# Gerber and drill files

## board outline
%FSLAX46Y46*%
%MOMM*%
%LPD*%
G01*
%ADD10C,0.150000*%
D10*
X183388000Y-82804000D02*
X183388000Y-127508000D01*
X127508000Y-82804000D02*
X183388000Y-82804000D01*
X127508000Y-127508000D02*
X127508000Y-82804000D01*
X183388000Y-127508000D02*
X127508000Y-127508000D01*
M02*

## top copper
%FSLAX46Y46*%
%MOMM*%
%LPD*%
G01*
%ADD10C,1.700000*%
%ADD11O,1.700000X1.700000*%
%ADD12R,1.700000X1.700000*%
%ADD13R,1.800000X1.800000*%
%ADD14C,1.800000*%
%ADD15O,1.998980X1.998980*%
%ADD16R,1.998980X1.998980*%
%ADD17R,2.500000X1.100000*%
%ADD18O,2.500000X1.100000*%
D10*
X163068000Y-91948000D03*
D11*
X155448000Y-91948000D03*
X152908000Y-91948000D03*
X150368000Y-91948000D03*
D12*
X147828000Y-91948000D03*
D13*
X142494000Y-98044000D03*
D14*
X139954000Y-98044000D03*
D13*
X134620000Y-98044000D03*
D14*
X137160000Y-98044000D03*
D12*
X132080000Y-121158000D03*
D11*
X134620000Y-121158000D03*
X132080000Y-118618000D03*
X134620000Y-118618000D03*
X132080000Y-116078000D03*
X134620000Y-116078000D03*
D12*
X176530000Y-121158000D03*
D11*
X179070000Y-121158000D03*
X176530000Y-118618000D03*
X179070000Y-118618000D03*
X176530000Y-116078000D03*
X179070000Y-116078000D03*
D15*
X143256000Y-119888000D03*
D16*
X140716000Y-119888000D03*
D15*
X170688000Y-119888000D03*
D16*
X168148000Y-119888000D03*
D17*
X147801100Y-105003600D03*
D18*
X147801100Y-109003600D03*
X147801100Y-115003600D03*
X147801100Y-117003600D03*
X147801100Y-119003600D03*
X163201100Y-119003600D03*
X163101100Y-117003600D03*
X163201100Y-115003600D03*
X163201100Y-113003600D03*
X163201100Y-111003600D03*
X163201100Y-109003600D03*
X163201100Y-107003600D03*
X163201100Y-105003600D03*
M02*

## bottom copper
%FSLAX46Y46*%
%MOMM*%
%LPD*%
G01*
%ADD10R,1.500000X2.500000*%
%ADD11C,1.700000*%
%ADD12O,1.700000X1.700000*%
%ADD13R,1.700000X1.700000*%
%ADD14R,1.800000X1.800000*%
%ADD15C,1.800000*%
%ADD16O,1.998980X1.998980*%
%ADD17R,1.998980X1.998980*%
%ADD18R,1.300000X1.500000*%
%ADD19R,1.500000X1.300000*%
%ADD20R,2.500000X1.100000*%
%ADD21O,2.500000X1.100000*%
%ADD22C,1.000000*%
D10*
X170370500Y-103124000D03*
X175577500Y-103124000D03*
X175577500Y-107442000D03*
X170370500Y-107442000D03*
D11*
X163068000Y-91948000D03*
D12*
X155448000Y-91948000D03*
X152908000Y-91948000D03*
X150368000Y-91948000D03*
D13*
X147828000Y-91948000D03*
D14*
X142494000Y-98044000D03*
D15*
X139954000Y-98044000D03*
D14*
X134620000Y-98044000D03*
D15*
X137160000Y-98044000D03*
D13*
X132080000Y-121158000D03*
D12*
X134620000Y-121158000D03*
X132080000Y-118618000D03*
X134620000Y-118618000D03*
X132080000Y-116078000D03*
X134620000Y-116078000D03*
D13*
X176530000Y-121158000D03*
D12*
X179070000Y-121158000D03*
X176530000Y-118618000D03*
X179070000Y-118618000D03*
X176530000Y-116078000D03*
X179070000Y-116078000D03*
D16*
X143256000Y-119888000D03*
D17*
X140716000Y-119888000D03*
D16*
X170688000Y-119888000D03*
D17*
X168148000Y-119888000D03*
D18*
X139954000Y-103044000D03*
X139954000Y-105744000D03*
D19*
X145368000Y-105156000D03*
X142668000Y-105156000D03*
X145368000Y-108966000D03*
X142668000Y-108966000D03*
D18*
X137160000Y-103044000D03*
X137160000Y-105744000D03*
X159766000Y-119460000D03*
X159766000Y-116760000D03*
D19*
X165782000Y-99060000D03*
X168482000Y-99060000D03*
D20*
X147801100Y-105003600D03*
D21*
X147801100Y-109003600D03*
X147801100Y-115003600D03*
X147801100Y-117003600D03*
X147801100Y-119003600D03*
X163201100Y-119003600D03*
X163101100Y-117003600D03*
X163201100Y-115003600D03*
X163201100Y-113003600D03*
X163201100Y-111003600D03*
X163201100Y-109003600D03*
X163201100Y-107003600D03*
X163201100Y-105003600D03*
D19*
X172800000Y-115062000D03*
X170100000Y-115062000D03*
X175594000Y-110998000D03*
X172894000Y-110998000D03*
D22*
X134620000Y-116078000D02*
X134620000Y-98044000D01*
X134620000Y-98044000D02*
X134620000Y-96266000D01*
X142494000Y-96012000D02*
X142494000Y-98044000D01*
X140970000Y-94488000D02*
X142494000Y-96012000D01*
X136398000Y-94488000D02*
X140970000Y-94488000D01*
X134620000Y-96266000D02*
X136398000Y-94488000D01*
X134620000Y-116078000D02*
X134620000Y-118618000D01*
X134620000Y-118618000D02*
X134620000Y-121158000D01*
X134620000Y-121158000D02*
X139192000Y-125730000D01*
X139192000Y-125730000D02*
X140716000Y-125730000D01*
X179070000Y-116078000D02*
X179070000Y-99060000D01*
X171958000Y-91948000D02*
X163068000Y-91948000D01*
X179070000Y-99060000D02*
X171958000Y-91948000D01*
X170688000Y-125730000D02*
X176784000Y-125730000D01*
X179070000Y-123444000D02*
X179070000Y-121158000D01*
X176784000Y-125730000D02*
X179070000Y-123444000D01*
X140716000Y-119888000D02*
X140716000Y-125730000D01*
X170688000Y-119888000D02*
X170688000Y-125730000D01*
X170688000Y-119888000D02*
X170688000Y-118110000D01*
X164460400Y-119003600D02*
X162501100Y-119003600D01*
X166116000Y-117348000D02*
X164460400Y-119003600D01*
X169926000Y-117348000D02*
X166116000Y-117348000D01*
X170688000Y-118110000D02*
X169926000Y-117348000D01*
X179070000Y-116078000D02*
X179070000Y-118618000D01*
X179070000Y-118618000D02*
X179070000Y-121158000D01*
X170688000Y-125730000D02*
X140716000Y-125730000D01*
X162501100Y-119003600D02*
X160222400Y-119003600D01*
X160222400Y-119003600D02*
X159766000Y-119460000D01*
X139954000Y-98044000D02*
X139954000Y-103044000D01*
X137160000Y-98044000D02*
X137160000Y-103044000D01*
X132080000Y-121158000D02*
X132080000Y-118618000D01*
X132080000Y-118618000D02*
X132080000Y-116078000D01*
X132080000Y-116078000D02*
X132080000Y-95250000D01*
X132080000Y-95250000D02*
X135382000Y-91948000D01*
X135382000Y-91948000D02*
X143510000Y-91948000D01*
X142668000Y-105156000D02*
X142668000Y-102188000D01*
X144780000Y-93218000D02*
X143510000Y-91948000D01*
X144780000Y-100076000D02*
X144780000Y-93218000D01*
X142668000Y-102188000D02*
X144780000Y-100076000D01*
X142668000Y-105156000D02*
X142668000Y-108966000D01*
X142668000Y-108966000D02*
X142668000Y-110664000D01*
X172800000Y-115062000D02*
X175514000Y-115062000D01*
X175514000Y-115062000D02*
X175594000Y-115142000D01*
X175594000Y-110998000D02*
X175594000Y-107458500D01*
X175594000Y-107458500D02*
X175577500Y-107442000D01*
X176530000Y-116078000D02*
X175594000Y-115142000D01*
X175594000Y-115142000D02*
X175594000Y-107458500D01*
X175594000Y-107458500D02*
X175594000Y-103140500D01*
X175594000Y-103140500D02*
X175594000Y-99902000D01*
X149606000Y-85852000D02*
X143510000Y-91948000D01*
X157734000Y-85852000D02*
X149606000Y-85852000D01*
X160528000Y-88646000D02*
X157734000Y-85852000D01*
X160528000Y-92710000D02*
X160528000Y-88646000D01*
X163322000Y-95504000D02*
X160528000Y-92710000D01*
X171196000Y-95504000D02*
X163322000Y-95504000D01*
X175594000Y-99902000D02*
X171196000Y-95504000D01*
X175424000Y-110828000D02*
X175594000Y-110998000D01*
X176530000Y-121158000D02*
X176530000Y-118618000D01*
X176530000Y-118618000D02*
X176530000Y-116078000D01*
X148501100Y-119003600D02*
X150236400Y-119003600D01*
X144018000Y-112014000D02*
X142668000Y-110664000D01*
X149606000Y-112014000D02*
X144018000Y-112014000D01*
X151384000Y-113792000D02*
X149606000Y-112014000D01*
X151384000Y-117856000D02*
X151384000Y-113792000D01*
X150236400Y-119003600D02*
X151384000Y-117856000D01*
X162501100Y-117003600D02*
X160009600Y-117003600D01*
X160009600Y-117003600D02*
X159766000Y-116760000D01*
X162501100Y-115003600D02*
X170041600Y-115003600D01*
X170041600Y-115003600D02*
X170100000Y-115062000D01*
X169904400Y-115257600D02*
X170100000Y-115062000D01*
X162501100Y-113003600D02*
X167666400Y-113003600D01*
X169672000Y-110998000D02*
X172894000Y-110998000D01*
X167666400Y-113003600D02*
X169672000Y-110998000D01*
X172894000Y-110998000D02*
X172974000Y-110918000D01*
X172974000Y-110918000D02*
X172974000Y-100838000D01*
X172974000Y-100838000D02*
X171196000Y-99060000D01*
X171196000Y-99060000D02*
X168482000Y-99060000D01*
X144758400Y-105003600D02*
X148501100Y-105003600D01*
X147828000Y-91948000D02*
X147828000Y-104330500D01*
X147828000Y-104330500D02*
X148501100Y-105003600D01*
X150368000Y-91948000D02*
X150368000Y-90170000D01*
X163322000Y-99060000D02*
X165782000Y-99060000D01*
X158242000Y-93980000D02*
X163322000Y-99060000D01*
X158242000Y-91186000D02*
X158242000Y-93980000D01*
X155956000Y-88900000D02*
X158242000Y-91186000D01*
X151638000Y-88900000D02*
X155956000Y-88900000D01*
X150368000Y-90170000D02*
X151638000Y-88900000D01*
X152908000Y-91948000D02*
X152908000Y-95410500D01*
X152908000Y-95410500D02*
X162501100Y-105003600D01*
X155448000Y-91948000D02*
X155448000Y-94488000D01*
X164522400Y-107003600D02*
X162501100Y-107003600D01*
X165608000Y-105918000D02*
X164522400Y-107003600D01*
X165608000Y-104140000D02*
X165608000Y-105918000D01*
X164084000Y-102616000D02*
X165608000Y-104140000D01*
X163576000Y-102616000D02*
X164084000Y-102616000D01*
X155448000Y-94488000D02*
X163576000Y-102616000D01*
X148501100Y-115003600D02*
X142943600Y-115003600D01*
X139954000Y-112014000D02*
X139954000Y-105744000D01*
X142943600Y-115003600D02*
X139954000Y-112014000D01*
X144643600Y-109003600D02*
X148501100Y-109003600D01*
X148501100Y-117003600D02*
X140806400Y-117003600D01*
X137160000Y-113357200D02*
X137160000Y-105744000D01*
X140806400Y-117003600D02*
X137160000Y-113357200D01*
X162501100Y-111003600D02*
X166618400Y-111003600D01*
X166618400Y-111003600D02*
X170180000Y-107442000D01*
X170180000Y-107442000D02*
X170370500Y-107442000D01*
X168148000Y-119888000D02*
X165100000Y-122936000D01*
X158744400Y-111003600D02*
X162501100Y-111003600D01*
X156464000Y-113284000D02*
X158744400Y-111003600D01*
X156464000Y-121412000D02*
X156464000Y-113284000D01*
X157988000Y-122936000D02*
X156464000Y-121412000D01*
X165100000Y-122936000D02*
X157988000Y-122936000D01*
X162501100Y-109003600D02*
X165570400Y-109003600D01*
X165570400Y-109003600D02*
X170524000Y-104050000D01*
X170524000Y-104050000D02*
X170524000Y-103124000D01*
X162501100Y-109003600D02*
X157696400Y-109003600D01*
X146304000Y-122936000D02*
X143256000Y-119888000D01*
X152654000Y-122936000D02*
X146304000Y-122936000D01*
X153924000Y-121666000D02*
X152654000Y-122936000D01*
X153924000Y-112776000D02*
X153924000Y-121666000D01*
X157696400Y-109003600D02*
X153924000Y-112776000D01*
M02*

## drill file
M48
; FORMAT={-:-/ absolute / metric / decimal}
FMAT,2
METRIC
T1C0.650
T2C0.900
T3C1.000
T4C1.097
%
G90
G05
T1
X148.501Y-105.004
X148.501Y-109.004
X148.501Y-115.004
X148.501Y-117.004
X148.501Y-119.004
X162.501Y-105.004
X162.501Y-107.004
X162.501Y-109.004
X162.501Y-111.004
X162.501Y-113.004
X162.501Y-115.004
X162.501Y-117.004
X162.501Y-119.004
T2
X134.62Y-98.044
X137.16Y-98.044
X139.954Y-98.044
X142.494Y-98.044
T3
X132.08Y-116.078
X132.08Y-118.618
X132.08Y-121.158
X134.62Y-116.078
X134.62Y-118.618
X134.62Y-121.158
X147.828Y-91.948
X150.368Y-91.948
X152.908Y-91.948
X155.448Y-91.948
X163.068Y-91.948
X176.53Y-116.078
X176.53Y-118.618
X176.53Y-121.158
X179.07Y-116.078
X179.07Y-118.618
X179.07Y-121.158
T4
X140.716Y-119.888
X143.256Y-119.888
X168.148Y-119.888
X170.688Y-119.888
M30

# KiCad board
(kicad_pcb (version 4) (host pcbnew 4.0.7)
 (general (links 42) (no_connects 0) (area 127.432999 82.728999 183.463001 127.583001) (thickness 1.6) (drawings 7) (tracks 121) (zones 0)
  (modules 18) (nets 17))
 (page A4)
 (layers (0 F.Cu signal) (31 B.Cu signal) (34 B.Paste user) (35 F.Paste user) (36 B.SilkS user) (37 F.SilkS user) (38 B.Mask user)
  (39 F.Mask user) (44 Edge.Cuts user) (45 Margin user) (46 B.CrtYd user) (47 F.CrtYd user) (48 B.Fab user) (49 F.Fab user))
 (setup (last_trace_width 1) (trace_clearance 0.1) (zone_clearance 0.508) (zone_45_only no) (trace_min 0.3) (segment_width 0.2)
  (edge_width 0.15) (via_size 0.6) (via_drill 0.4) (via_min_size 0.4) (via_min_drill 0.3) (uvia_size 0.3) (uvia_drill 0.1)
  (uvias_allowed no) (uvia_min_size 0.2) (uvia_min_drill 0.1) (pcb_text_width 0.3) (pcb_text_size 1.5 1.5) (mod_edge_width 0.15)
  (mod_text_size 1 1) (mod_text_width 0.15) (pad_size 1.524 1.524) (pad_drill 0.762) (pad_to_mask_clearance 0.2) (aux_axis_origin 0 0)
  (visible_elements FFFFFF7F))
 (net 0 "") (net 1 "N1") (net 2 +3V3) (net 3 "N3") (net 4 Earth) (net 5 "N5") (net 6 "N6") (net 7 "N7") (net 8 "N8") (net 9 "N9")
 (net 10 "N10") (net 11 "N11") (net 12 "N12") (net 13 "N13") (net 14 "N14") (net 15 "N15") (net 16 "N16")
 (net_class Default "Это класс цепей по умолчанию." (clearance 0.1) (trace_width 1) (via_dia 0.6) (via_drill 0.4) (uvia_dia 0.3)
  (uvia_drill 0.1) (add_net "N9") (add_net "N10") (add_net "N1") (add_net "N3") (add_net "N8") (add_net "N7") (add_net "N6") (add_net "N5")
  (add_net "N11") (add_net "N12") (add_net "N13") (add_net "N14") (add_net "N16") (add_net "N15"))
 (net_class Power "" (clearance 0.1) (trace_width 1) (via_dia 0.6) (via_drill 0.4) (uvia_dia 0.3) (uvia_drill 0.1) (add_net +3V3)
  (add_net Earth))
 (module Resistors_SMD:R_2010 (layer B.Cu) (at 172.974 103.124)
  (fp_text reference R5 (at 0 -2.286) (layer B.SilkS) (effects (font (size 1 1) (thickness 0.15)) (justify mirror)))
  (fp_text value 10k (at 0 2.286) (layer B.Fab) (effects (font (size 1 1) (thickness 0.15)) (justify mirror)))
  (pad 1 smd rect (at -2.6035 0) (size 1.5 2.5) (layers B.Cu B.Paste B.Mask) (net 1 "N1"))
  (pad 2 smd rect (at 2.6035 0) (size 1.5 2.5) (layers B.Cu B.Paste B.Mask) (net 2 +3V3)))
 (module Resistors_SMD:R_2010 (layer B.Cu) (at 172.974 107.442 180)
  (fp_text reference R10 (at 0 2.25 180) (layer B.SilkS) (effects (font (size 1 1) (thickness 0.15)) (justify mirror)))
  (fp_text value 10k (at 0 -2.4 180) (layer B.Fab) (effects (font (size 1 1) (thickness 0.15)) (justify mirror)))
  (pad 1 smd rect (at -2.6035 0 180) (size 1.5 2.5) (layers B.Cu B.Paste B.Mask) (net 2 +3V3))
  (pad 2 smd rect (at 2.6035 0 180) (size 1.5 2.5) (layers B.Cu B.Paste B.Mask) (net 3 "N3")))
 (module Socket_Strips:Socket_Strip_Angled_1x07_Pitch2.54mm (layer F.Cu) (at 163.068 91.948 270)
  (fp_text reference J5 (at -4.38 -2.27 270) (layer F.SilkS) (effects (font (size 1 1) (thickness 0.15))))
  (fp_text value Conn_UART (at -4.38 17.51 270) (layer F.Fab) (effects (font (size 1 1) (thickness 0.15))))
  (pad 7 thru_hole circle (at 0 0 270) (size 1.7 1.7) (drill 1) (layers *.Cu *.Mask) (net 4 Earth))
  (pad 4 thru_hole oval (at 0 7.62 270) (size 1.7 1.7) (drill 1) (layers *.Cu *.Mask) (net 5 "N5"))
  (pad 3 thru_hole oval (at 0 10.16 270) (size 1.7 1.7) (drill 1) (layers *.Cu *.Mask) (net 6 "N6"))
  (pad 2 thru_hole oval (at 0 12.7 270) (size 1.7 1.7) (drill 1) (layers *.Cu *.Mask) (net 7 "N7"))
  (pad 1 thru_hole rect (at 0 15.24 270) (size 1.7 1.7) (drill 1) (layers *.Cu *.Mask) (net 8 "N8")))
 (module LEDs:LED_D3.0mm (layer F.Cu) (at 142.494 98.044 180)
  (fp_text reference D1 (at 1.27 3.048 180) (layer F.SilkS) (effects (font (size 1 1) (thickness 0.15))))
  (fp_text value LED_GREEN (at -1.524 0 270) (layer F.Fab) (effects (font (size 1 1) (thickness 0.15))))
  (pad 1 thru_hole rect (at 0 0 180) (size 1.8 1.8) (drill 0.9) (layers *.Cu *.Mask) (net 4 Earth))
  (pad 2 thru_hole circle (at 2.54 0 180) (size 1.8 1.8) (drill 0.9) (layers *.Cu *.Mask) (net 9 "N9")))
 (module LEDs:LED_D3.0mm (layer F.Cu) (at 134.62 98.044)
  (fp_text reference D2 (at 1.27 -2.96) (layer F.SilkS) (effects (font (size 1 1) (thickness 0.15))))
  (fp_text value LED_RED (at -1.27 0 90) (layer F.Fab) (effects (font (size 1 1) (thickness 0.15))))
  (pad 1 thru_hole rect (at 0 0) (size 1.8 1.8) (drill 0.9) (layers *.Cu *.Mask) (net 4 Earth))
  (pad 2 thru_hole circle (at 2.54 0) (size 1.8 1.8) (drill 0.9) (layers *.Cu *.Mask) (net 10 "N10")))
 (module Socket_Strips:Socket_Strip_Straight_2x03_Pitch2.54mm (layer F.Cu) (at 132.08 121.158 180)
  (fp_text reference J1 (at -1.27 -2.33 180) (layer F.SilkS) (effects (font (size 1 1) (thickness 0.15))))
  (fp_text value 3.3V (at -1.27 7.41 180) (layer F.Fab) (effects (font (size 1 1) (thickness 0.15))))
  (pad 1 thru_hole rect (at 0 0 180) (size 1.7 1.7) (drill 1) (layers *.Cu *.Mask) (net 2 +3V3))
  (pad 2 thru_hole oval (at -2.54 0 180) (size 1.7 1.7) (drill 1) (layers *.Cu *.Mask) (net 4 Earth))
  (pad 3 thru_hole oval (at 0 2.54 180) (size 1.7 1.7) (drill 1) (layers *.Cu *.Mask) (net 2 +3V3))
  (pad 4 thru_hole oval (at -2.54 2.54 180) (size 1.7 1.7) (drill 1) (layers *.Cu *.Mask) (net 4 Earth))
  (pad 5 thru_hole oval (at 0 5.08 180) (size 1.7 1.7) (drill 1) (layers *.Cu *.Mask) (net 2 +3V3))
  (pad 6 thru_hole oval (at -2.54 5.08 180) (size 1.7 1.7) (drill 1) (layers *.Cu *.Mask) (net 4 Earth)))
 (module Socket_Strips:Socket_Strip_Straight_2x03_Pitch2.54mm (layer F.Cu) (at 176.53 121.158 180)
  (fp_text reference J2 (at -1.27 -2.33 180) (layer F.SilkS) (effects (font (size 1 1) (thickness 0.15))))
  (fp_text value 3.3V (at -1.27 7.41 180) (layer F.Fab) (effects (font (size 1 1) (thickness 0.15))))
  (pad 1 thru_hole rect (at 0 0 180) (size 1.7 1.7) (drill 1) (layers *.Cu *.Mask) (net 2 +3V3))
  (pad 2 thru_hole oval (at -2.54 0 180) (size 1.7 1.7) (drill 1) (layers *.Cu *.Mask) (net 4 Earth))
  (pad 3 thru_hole oval (at 0 2.54 180) (size 1.7 1.7) (drill 1) (layers *.Cu *.Mask) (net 2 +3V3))
  (pad 4 thru_hole oval (at -2.54 2.54 180) (size 1.7 1.7) (drill 1) (layers *.Cu *.Mask) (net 4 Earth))
  (pad 5 thru_hole oval (at 0 5.08 180) (size 1.7 1.7) (drill 1) (layers *.Cu *.Mask) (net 2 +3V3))
  (pad 6 thru_hole oval (at -2.54 5.08 180) (size 1.7 1.7) (drill 1) (layers *.Cu *.Mask) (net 4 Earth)))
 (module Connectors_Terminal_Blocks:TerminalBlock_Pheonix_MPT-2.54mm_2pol (layer F.Cu) (at 140.716 119.888)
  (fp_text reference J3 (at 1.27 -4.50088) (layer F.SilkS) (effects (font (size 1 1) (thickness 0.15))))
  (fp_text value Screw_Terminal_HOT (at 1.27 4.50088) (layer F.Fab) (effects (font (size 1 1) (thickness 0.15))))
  (pad 2 thru_hole oval (at 2.54 0) (size 1.99898 1.99898) (drill 1.09728) (layers *.Cu *.Mask) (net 1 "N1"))
  (pad 1 thru_hole rect (at 0 0) (size 1.99898 1.99898) (drill 1.09728) (layers *.Cu *.Mask) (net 4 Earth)))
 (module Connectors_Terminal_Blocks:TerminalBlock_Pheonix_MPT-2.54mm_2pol (layer F.Cu) (at 168.148 119.888)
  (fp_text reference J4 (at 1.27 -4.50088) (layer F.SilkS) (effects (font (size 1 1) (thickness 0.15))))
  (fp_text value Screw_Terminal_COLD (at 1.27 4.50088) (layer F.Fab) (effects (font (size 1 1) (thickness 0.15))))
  (pad 2 thru_hole oval (at 2.54 0) (size 1.99898 1.99898) (drill 1.09728) (layers *.Cu *.Mask) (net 4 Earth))
  (pad 1 thru_hole rect (at 0 0) (size 1.99898 1.99898) (drill 1.09728) (layers *.Cu *.Mask) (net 3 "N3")))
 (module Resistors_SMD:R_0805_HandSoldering (layer B.Cu) (at 139.954 104.394 270)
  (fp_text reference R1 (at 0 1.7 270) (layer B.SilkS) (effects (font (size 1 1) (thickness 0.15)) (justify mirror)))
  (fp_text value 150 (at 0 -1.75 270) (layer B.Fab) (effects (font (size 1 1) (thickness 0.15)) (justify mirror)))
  (pad 1 smd rect (at -1.35 0 270) (size 1.5 1.3) (layers B.Cu B.Paste B.Mask) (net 9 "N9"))
  (pad 2 smd rect (at 1.35 0 270) (size 1.5 1.3) (layers B.Cu B.Paste B.Mask) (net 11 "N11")))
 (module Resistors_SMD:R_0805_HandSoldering (layer B.Cu) (at 144.018 105.156 180)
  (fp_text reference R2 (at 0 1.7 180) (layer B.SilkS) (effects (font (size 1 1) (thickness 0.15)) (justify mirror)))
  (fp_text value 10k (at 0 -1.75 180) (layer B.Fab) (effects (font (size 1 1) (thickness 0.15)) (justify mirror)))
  (pad 1 smd rect (at -1.35 0 180) (size 1.5 1.3) (layers B.Cu B.Paste B.Mask) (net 8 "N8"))
  (pad 2 smd rect (at 1.35 0 180) (size 1.5 1.3) (layers B.Cu B.Paste B.Mask) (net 2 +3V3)))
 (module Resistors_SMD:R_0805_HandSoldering (layer B.Cu) (at 144.018 108.966 180)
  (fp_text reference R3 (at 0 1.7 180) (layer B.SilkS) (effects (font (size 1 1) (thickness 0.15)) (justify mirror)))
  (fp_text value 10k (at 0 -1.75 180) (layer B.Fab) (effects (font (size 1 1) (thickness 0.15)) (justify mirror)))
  (pad 1 smd rect (at -1.35 0 180) (size 1.5 1.3) (layers B.Cu B.Paste B.Mask) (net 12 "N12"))
  (pad 2 smd rect (at 1.35 0 180) (size 1.5 1.3) (layers B.Cu B.Paste B.Mask) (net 2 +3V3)))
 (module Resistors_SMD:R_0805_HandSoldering (layer B.Cu) (at 137.16 104.394 270)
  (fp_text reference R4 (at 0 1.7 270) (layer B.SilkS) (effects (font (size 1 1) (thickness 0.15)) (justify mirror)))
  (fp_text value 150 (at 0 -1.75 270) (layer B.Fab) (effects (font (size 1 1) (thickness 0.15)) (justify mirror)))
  (pad 1 smd rect (at -1.35 0 270) (size 1.5 1.3) (layers B.Cu B.Paste B.Mask) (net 10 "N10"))
  (pad 2 smd rect (at 1.35 0 270) (size 1.5 1.3) (layers B.Cu B.Paste B.Mask) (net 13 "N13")))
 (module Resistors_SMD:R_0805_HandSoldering (layer B.Cu) (at 159.766 118.11 90)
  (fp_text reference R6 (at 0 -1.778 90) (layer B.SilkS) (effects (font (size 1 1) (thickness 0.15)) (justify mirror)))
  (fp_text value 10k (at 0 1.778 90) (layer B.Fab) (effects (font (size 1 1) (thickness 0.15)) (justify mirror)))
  (pad 1 smd rect (at -1.35 0 90) (size 1.5 1.3) (layers B.Cu B.Paste B.Mask) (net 4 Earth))
  (pad 2 smd rect (at 1.35 0 90) (size 1.5 1.3) (layers B.Cu B.Paste B.Mask) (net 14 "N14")))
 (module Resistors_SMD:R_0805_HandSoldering (layer B.Cu) (at 167.132 99.06)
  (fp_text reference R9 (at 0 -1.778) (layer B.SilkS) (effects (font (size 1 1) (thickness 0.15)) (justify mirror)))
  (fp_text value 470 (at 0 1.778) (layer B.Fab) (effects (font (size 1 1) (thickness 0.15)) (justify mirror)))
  (pad 1 smd rect (at -1.35 0) (size 1.5 1.3) (layers B.Cu B.Paste B.Mask) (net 7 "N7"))
  (pad 2 smd rect (at 1.35 0) (size 1.5 1.3) (layers B.Cu B.Paste B.Mask) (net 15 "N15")))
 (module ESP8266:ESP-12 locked (layer F.Cu) (at 148.5011 105.0036)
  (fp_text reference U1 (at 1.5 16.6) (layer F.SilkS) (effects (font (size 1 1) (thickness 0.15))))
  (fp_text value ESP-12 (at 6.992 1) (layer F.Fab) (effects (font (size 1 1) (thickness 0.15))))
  (pad 1 thru_hole rect (at 0 0) (size 2.5 1.1) (drill 0.65 (offset -0.7 0)) (layers *.Cu *.Mask F.SilkS) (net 8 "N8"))
  (pad 3 thru_hole oval (at 0 4) (size 2.5 1.1) (drill 0.65 (offset -0.7 0)) (layers *.Cu *.Mask F.SilkS) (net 12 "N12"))
  (pad 6 thru_hole oval (at 0 10) (size 2.5 1.1) (drill 0.65 (offset -0.7 0)) (layers *.Cu *.Mask F.SilkS) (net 11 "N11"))
  (pad 7 thru_hole oval (at 0 12) (size 2.5 1.1) (drill 0.65 (offset -0.7 0)) (layers *.Cu *.Mask F.SilkS) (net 13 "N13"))
  (pad 8 thru_hole oval (at 0 14) (size 2.5 1.1) (drill 0.65 (offset -0.7 0)) (layers *.Cu *.Mask F.SilkS) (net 2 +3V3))
  (pad 9 thru_hole oval (at 14 14) (size 2.5 1.1) (drill 0.65 (offset 0.7 0)) (layers *.Cu *.Mask F.SilkS) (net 4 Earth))
  (pad 10 thru_hole oval (at 14 12) (size 2.5 1.1) (drill 0.65 (offset 0.6 0)) (layers *.Cu *.Mask F.SilkS) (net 14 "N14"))
  (pad 11 thru_hole oval (at 14 10) (size 2.5 1.1) (drill 0.65 (offset 0.7 0)) (layers *.Cu *.Mask F.SilkS) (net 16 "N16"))
  (pad 12 thru_hole oval (at 14 8) (size 2.5 1.1) (drill 0.65 (offset 0.7 0)) (layers *.Cu *.Mask F.SilkS) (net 15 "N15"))
  (pad 13 thru_hole oval (at 14 6) (size 2.5 1.1) (drill 0.65 (offset 0.7 0)) (layers *.Cu *.Mask F.SilkS) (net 3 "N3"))
  (pad 14 thru_hole oval (at 14 4) (size 2.5 1.1) (drill 0.65 (offset 0.7 0)) (layers *.Cu *.Mask F.SilkS) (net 1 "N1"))
  (pad 15 thru_hole oval (at 14 2) (size 2.5 1.1) (drill 0.65 (offset 0.7 0)) (layers *.Cu *.Mask F.SilkS) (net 5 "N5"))
  (pad 16 thru_hole oval (at 14 0) (size 2.5 1.1) (drill 0.65 (offset 0.7 0)) (layers *.Cu *.Mask F.SilkS) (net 6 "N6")))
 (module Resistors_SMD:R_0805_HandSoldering (layer B.Cu) (at 171.45 115.062 180)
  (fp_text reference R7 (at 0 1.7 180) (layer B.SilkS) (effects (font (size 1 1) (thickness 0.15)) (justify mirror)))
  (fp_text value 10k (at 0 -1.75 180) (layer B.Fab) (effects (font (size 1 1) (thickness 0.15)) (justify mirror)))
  (pad 1 smd rect (at -1.35 0 180) (size 1.5 1.3) (layers B.Cu B.Paste B.Mask) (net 2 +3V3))
  (pad 2 smd rect (at 1.35 0 180) (size 1.5 1.3) (layers B.Cu B.Paste B.Mask) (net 16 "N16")))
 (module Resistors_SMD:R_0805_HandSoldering (layer B.Cu) (at 174.244 110.998 180)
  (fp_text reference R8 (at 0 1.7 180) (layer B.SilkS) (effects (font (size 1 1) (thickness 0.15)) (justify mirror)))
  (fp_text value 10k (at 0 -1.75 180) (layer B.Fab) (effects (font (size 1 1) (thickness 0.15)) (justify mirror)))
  (pad 1 smd rect (at -1.35 0 180) (size 1.5 1.3) (layers B.Cu B.Paste B.Mask) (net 2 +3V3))
  (pad 2 smd rect (at 1.35 0 180) (size 1.5 1.3) (layers B.Cu B.Paste B.Mask) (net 15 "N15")))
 (gr_line (start 183.388 82.804) (end 183.388 127.508) (angle 90) (layer Edge.Cuts) (width 0.15))
 (gr_line (start 127.508 82.804) (end 183.388 82.804) (angle 90) (layer Edge.Cuts) (width 0.15))
 (gr_line (start 127.508 127.508) (end 127.508 82.804) (angle 90) (layer Edge.Cuts) (width 0.15))
 (gr_line (start 183.388 127.508) (end 127.508 127.508) (angle 90) (layer Edge.Cuts) (width 0.15))
 (segment (start 134.62 116.078) (end 134.62 98.044) (width 1) (layer B.Cu) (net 4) (status 30))
 (segment (start 134.62 98.044) (end 134.62 96.266) (width 1) (layer B.Cu) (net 4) (status 10))
 (segment (start 142.494 96.012) (end 142.494 98.044) (width 1) (layer B.Cu) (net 4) (status 20))
 (segment (start 140.97 94.488) (end 142.494 96.012) (width 1) (layer B.Cu) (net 4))
 (segment (start 136.398 94.488) (end 140.97 94.488) (width 1) (layer B.Cu) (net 4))
 (segment (start 134.62 96.266) (end 136.398 94.488) (width 1) (layer B.Cu) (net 4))
 (segment (start 134.62 116.078) (end 134.62 118.618) (width 1) (layer B.Cu) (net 4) (status 30))
 (segment (start 134.62 118.618) (end 134.62 121.158) (width 1) (layer B.Cu) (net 4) (status 30))
 (segment (start 134.62 121.158) (end 139.192 125.73) (width 1) (layer B.Cu) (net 4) (status 10))
 (segment (start 139.192 125.73) (end 140.716 125.73) (width 1) (layer B.Cu) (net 4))
 (segment (start 179.07 116.078) (end 179.07 99.06) (width 1) (layer B.Cu) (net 4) (status 10))
 (segment (start 171.958 91.948) (end 163.068 91.948) (width 1) (layer B.Cu) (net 4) (status 20))
 (segment (start 179.07 99.06) (end 171.958 91.948) (width 1) (layer B.Cu) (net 4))
 (segment (start 170.688 125.73) (end 176.784 125.73) (width 1) (layer B.Cu) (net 4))
 (segment (start 179.07 123.444) (end 179.07 121.158) (width 1) (layer B.Cu) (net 4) (status 20))
 (segment (start 176.784 125.73) (end 179.07 123.444) (width 1) (layer B.Cu) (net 4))
 (segment (start 140.716 119.888) (end 140.716 125.73) (width 1) (layer B.Cu) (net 4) (status 10))
 (segment (start 170.688 119.888) (end 170.688 125.73) (width 1) (layer B.Cu) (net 4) (status 10))
 (segment (start 170.688 119.888) (end 170.688 118.11) (width 1) (layer B.Cu) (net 4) (status 10))
 (segment (start 164.4604 119.0036) (end 162.5011 119.0036) (width 1) (layer B.Cu) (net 4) (status 20))
 (segment (start 166.116 117.348) (end 164.4604 119.0036) (width 1) (layer B.Cu) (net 4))
 (segment (start 169.926 117.348) (end 166.116 117.348) (width 1) (layer B.Cu) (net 4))
 (segment (start 170.688 118.11) (end 169.926 117.348) (width 1) (layer B.Cu) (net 4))
 (segment (start 179.07 116.078) (end 179.07 118.618) (width 1) (layer B.Cu) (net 4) (status 30))
 (segment (start 179.07 118.618) (end 179.07 121.158) (width 1) (layer B.Cu) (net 4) (status 30))
 (segment (start 170.688 125.73) (end 140.716 125.73) (width 1) (layer B.Cu) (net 4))
 (segment (start 162.5011 119.0036) (end 160.2224 119.0036) (width 1) (layer B.Cu) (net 4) (status 30))
 (segment (start 160.2224 119.0036) (end 159.766 119.46) (width 1) (layer B.Cu) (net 4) (status 30))
 (segment (start 139.954 98.044) (end 139.954 103.044) (width 1) (layer B.Cu) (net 9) (status 30))
 (segment (start 137.16 98.044) (end 137.16 103.044) (width 1) (layer B.Cu) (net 10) (status 30))
 (segment (start 132.08 121.158) (end 132.08 118.618) (width 1) (layer B.Cu) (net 2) (status 30))
 (segment (start 132.08 118.618) (end 132.08 116.078) (width 1) (layer B.Cu) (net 2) (status 30))
 (segment (start 132.08 116.078) (end 132.08 95.25) (width 1) (layer B.Cu) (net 2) (status 10))
 (segment (start 132.08 95.25) (end 135.382 91.948) (width 1) (layer B.Cu) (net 2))
 (segment (start 135.382 91.948) (end 143.51 91.948) (width 1) (layer B.Cu) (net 2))
 (segment (start 142.668 105.156) (end 142.668 102.188) (width 1) (layer B.Cu) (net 2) (status 10))
 (segment (start 144.78 93.218) (end 143.51 91.948) (width 1) (layer B.Cu) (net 2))
 (segment (start 144.78 100.076) (end 144.78 93.218) (width 1) (layer B.Cu) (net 2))
 (segment (start 142.668 102.188) (end 144.78 100.076) (width 1) (layer B.Cu) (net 2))
 (segment (start 142.668 105.156) (end 142.668 108.966) (width 1) (layer B.Cu) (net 2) (status 30))
 (segment (start 142.668 108.966) (end 142.668 110.664) (width 1) (layer B.Cu) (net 2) (status 10))
 (segment (start 172.8 115.062) (end 175.514 115.062) (width 1) (layer B.Cu) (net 2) (status 10))
 (segment (start 175.514 115.062) (end 175.594 115.142) (width 1) (layer B.Cu) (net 2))
 (segment (start 175.594 110.998) (end 175.594 107.4585) (width 1) (layer B.Cu) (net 2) (status 30))
 (segment (start 175.594 107.4585) (end 175.5775 107.442) (width 1) (layer B.Cu) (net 2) (status 30))
 (segment (start 176.53 116.078) (end 175.594 115.142) (width 1) (layer B.Cu) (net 2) (status 10))
 (segment (start 175.594 115.142) (end 175.594 107.4585) (width 1) (layer B.Cu) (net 2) (status 20))
 (segment (start 175.594 107.4585) (end 175.594 103.1405) (width 1) (layer B.Cu) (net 2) (status 30))
 (segment (start 175.594 103.1405) (end 175.594 99.902) (width 1) (layer B.Cu) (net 2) (status 10))
 (segment (start 149.606 85.852) (end 143.51 91.948) (width 1) (layer B.Cu) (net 2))
 (segment (start 157.734 85.852) (end 149.606 85.852) (width 1) (layer B.Cu) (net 2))
 (segment (start 160.528 88.646) (end 157.734 85.852) (width 1) (layer B.Cu) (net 2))
 (segment (start 160.528 92.71) (end 160.528 88.646) (width 1) (layer B.Cu) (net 2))
 (segment (start 163.322 95.504) (end 160.528 92.71) (width 1) (layer B.Cu) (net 2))
 (segment (start 171.196 95.504) (end 163.322 95.504) (width 1) (layer B.Cu) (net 2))
 (segment (start 175.594 99.902) (end 171.196 95.504) (width 1) (layer B.Cu) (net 2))
 (segment (start 175.424 110.828) (end 175.594 110.998) (width 1) (layer B.Cu) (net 2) (status 30))
 (segment (start 176.53 121.158) (end 176.53 118.618) (width 1) (layer B.Cu) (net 2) (status 30))
 (segment (start 176.53 118.618) (end 176.53 116.078) (width 1) (layer B.Cu) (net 2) (status 30))
 (segment (start 148.5011 119.0036) (end 150.2364 119.0036) (width 1) (layer B.Cu) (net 2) (status 10))
 (segment (start 144.018 112.014) (end 142.668 110.664) (width 1) (layer B.Cu) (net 2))
 (segment (start 149.606 112.014) (end 144.018 112.014) (width 1) (layer B.Cu) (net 2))
 (segment (start 151.384 113.792) (end 149.606 112.014) (width 1) (layer B.Cu) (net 2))
 (segment (start 151.384 117.856) (end 151.384 113.792) (width 1) (layer B.Cu) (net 2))
 (segment (start 150.2364 119.0036) (end 151.384 117.856) (width 1) (layer B.Cu) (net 2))
 (segment (start 162.5011 117.0036) (end 160.0096 117.0036) (width 1) (layer B.Cu) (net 14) (status 30))
 (segment (start 160.0096 117.0036) (end 159.766 116.76) (width 1) (layer B.Cu) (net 14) (status 30))
 (segment (start 162.5011 115.0036) (end 170.0416 115.0036) (width 1) (layer B.Cu) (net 16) (status 30))
 (segment (start 170.0416 115.0036) (end 170.1 115.062) (width 1) (layer B.Cu) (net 16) (status 30))
 (segment (start 169.9044 115.2576) (end 170.1 115.062) (width 1) (layer B.Cu) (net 16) (status 30))
 (segment (start 162.5011 113.0036) (end 167.6664 113.0036) (width 1) (layer B.Cu) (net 15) (status 10))
 (segment (start 169.672 110.998) (end 172.894 110.998) (width 1) (layer B.Cu) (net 15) (status 20))
 (segment (start 167.6664 113.0036) (end 169.672 110.998) (width 1) (layer B.Cu) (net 15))
 (segment (start 172.894 110.998) (end 172.974 110.918) (width 1) (layer B.Cu) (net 15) (status 30))
 (segment (start 172.974 110.918) (end 172.974 100.838) (width 1) (layer B.Cu) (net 15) (status 10))
 (segment (start 172.974 100.838) (end 171.196 99.06) (width 1) (layer B.Cu) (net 15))
 (segment (start 171.196 99.06) (end 168.482 99.06) (width 1) (layer B.Cu) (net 15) (status 20))
 (segment (start 144.7584 105.0036) (end 148.5011 105.0036) (width 1) (layer B.Cu) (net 8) (status 30))
 (segment (start 147.828 91.948) (end 147.828 104.3305) (width 1) (layer B.Cu) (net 8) (status 10))
 (segment (start 147.828 104.3305) (end 148.5011 105.0036) (width 1) (layer B.Cu) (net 8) (status 20))
 (segment (start 150.368 91.948) (end 150.368 90.17) (width 1) (layer B.Cu) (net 7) (status 10))
 (segment (start 163.322 99.06) (end 165.782 99.06) (width 1) (layer B.Cu) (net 7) (status 20))
 (segment (start 158.242 93.98) (end 163.322 99.06) (width 1) (layer B.Cu) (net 7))
 (segment (start 158.242 91.186) (end 158.242 93.98) (width 1) (layer B.Cu) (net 7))
 (segment (start 155.956 88.9) (end 158.242 91.186) (width 1) (layer B.Cu) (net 7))
 (segment (start 151.638 88.9) (end 155.956 88.9) (width 1) (layer B.Cu) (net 7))
 (segment (start 150.368 90.17) (end 151.638 88.9) (width 1) (layer B.Cu) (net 7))
 (segment (start 152.908 91.948) (end 152.908 95.4105) (width 1) (layer B.Cu) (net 6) (status 10))
 (segment (start 152.908 95.4105) (end 162.5011 105.0036) (width 1) (layer B.Cu) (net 6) (status 20))
 (segment (start 155.448 91.948) (end 155.448 94.488) (width 1) (layer B.Cu) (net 5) (status 10))
 (segment (start 164.5224 107.0036) (end 162.5011 107.0036) (width 1) (layer B.Cu) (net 5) (status 20))
 (segment (start 165.608 105.918) (end 164.5224 107.0036) (width 1) (layer B.Cu) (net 5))
 (segment (start 165.608 104.14) (end 165.608 105.918) (width 1) (layer B.Cu) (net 5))
 (segment (start 164.084 102.616) (end 165.608 104.14) (width 1) (layer B.Cu) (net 5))
 (segment (start 163.576 102.616) (end 164.084 102.616) (width 1) (layer B.Cu) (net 5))
 (segment (start 155.448 94.488) (end 163.576 102.616) (width 1) (layer B.Cu) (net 5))
 (segment (start 148.5011 115.0036) (end 142.9436 115.0036) (width 1) (layer B.Cu) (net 11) (status 10))
 (segment (start 139.954 112.014) (end 139.954 105.744) (width 1) (layer B.Cu) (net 11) (status 20))
 (segment (start 142.9436 115.0036) (end 139.954 112.014) (width 1) (layer B.Cu) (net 11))
 (segment (start 144.6436 109.0036) (end 148.5011 109.0036) (width 1) (layer B.Cu) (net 12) (status 30))
 (segment (start 148.5011 117.0036) (end 140.8064 117.0036) (width 1) (layer B.Cu) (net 13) (status 10))
 (segment (start 137.16 113.3572) (end 137.16 105.744) (width 1) (layer B.Cu) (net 13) (status 20))
 (segment (start 140.8064 117.0036) (end 137.16 113.3572) (width 1) (layer B.Cu) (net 13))
 (segment (start 162.5011 111.0036) (end 166.6184 111.0036) (width 1) (layer B.Cu) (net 3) (status 10))
 (segment (start 166.6184 111.0036) (end 170.18 107.442) (width 1) (layer B.Cu) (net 3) (status 20))
 (segment (start 170.18 107.442) (end 170.3705 107.442) (width 1) (layer B.Cu) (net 3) (status 30))
 (segment (start 168.148 119.888) (end 165.1 122.936) (width 1) (layer B.Cu) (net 3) (status 10))
 (segment (start 158.7444 111.0036) (end 162.5011 111.0036) (width 1) (layer B.Cu) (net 3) (status 20))
 (segment (start 156.464 113.284) (end 158.7444 111.0036) (width 1) (layer B.Cu) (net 3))
 (segment (start 156.464 121.412) (end 156.464 113.284) (width 1) (layer B.Cu) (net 3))
 (segment (start 157.988 122.936) (end 156.464 121.412) (width 1) (layer B.Cu) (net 3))
 (segment (start 165.1 122.936) (end 157.988 122.936) (width 1) (layer B.Cu) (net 3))
 (segment (start 162.5011 109.0036) (end 165.5704 109.0036) (width 1) (layer B.Cu) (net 1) (status 10))
 (segment (start 165.5704 109.0036) (end 170.524 104.05) (width 1) (layer B.Cu) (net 1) (status 20))
 (segment (start 170.524 104.05) (end 170.524 103.124) (width 1) (layer B.Cu) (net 1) (status 30))
 (segment (start 162.5011 109.0036) (end 157.6964 109.0036) (width 1) (layer B.Cu) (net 1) (status 10))
 (segment (start 146.304 122.936) (end 143.256 119.888) (width 1) (layer B.Cu) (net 1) (status 20))
 (segment (start 152.654 122.936) (end 146.304 122.936) (width 1) (layer B.Cu) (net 1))
 (segment (start 153.924 121.666) (end 152.654 122.936) (width 1) (layer B.Cu) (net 1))
 (segment (start 153.924 112.776) (end 153.924 121.666) (width 1) (layer B.Cu) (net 1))
 (segment (start 157.6964 109.0036) (end 153.924 112.776) (width 1) (layer B.Cu) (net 1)))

